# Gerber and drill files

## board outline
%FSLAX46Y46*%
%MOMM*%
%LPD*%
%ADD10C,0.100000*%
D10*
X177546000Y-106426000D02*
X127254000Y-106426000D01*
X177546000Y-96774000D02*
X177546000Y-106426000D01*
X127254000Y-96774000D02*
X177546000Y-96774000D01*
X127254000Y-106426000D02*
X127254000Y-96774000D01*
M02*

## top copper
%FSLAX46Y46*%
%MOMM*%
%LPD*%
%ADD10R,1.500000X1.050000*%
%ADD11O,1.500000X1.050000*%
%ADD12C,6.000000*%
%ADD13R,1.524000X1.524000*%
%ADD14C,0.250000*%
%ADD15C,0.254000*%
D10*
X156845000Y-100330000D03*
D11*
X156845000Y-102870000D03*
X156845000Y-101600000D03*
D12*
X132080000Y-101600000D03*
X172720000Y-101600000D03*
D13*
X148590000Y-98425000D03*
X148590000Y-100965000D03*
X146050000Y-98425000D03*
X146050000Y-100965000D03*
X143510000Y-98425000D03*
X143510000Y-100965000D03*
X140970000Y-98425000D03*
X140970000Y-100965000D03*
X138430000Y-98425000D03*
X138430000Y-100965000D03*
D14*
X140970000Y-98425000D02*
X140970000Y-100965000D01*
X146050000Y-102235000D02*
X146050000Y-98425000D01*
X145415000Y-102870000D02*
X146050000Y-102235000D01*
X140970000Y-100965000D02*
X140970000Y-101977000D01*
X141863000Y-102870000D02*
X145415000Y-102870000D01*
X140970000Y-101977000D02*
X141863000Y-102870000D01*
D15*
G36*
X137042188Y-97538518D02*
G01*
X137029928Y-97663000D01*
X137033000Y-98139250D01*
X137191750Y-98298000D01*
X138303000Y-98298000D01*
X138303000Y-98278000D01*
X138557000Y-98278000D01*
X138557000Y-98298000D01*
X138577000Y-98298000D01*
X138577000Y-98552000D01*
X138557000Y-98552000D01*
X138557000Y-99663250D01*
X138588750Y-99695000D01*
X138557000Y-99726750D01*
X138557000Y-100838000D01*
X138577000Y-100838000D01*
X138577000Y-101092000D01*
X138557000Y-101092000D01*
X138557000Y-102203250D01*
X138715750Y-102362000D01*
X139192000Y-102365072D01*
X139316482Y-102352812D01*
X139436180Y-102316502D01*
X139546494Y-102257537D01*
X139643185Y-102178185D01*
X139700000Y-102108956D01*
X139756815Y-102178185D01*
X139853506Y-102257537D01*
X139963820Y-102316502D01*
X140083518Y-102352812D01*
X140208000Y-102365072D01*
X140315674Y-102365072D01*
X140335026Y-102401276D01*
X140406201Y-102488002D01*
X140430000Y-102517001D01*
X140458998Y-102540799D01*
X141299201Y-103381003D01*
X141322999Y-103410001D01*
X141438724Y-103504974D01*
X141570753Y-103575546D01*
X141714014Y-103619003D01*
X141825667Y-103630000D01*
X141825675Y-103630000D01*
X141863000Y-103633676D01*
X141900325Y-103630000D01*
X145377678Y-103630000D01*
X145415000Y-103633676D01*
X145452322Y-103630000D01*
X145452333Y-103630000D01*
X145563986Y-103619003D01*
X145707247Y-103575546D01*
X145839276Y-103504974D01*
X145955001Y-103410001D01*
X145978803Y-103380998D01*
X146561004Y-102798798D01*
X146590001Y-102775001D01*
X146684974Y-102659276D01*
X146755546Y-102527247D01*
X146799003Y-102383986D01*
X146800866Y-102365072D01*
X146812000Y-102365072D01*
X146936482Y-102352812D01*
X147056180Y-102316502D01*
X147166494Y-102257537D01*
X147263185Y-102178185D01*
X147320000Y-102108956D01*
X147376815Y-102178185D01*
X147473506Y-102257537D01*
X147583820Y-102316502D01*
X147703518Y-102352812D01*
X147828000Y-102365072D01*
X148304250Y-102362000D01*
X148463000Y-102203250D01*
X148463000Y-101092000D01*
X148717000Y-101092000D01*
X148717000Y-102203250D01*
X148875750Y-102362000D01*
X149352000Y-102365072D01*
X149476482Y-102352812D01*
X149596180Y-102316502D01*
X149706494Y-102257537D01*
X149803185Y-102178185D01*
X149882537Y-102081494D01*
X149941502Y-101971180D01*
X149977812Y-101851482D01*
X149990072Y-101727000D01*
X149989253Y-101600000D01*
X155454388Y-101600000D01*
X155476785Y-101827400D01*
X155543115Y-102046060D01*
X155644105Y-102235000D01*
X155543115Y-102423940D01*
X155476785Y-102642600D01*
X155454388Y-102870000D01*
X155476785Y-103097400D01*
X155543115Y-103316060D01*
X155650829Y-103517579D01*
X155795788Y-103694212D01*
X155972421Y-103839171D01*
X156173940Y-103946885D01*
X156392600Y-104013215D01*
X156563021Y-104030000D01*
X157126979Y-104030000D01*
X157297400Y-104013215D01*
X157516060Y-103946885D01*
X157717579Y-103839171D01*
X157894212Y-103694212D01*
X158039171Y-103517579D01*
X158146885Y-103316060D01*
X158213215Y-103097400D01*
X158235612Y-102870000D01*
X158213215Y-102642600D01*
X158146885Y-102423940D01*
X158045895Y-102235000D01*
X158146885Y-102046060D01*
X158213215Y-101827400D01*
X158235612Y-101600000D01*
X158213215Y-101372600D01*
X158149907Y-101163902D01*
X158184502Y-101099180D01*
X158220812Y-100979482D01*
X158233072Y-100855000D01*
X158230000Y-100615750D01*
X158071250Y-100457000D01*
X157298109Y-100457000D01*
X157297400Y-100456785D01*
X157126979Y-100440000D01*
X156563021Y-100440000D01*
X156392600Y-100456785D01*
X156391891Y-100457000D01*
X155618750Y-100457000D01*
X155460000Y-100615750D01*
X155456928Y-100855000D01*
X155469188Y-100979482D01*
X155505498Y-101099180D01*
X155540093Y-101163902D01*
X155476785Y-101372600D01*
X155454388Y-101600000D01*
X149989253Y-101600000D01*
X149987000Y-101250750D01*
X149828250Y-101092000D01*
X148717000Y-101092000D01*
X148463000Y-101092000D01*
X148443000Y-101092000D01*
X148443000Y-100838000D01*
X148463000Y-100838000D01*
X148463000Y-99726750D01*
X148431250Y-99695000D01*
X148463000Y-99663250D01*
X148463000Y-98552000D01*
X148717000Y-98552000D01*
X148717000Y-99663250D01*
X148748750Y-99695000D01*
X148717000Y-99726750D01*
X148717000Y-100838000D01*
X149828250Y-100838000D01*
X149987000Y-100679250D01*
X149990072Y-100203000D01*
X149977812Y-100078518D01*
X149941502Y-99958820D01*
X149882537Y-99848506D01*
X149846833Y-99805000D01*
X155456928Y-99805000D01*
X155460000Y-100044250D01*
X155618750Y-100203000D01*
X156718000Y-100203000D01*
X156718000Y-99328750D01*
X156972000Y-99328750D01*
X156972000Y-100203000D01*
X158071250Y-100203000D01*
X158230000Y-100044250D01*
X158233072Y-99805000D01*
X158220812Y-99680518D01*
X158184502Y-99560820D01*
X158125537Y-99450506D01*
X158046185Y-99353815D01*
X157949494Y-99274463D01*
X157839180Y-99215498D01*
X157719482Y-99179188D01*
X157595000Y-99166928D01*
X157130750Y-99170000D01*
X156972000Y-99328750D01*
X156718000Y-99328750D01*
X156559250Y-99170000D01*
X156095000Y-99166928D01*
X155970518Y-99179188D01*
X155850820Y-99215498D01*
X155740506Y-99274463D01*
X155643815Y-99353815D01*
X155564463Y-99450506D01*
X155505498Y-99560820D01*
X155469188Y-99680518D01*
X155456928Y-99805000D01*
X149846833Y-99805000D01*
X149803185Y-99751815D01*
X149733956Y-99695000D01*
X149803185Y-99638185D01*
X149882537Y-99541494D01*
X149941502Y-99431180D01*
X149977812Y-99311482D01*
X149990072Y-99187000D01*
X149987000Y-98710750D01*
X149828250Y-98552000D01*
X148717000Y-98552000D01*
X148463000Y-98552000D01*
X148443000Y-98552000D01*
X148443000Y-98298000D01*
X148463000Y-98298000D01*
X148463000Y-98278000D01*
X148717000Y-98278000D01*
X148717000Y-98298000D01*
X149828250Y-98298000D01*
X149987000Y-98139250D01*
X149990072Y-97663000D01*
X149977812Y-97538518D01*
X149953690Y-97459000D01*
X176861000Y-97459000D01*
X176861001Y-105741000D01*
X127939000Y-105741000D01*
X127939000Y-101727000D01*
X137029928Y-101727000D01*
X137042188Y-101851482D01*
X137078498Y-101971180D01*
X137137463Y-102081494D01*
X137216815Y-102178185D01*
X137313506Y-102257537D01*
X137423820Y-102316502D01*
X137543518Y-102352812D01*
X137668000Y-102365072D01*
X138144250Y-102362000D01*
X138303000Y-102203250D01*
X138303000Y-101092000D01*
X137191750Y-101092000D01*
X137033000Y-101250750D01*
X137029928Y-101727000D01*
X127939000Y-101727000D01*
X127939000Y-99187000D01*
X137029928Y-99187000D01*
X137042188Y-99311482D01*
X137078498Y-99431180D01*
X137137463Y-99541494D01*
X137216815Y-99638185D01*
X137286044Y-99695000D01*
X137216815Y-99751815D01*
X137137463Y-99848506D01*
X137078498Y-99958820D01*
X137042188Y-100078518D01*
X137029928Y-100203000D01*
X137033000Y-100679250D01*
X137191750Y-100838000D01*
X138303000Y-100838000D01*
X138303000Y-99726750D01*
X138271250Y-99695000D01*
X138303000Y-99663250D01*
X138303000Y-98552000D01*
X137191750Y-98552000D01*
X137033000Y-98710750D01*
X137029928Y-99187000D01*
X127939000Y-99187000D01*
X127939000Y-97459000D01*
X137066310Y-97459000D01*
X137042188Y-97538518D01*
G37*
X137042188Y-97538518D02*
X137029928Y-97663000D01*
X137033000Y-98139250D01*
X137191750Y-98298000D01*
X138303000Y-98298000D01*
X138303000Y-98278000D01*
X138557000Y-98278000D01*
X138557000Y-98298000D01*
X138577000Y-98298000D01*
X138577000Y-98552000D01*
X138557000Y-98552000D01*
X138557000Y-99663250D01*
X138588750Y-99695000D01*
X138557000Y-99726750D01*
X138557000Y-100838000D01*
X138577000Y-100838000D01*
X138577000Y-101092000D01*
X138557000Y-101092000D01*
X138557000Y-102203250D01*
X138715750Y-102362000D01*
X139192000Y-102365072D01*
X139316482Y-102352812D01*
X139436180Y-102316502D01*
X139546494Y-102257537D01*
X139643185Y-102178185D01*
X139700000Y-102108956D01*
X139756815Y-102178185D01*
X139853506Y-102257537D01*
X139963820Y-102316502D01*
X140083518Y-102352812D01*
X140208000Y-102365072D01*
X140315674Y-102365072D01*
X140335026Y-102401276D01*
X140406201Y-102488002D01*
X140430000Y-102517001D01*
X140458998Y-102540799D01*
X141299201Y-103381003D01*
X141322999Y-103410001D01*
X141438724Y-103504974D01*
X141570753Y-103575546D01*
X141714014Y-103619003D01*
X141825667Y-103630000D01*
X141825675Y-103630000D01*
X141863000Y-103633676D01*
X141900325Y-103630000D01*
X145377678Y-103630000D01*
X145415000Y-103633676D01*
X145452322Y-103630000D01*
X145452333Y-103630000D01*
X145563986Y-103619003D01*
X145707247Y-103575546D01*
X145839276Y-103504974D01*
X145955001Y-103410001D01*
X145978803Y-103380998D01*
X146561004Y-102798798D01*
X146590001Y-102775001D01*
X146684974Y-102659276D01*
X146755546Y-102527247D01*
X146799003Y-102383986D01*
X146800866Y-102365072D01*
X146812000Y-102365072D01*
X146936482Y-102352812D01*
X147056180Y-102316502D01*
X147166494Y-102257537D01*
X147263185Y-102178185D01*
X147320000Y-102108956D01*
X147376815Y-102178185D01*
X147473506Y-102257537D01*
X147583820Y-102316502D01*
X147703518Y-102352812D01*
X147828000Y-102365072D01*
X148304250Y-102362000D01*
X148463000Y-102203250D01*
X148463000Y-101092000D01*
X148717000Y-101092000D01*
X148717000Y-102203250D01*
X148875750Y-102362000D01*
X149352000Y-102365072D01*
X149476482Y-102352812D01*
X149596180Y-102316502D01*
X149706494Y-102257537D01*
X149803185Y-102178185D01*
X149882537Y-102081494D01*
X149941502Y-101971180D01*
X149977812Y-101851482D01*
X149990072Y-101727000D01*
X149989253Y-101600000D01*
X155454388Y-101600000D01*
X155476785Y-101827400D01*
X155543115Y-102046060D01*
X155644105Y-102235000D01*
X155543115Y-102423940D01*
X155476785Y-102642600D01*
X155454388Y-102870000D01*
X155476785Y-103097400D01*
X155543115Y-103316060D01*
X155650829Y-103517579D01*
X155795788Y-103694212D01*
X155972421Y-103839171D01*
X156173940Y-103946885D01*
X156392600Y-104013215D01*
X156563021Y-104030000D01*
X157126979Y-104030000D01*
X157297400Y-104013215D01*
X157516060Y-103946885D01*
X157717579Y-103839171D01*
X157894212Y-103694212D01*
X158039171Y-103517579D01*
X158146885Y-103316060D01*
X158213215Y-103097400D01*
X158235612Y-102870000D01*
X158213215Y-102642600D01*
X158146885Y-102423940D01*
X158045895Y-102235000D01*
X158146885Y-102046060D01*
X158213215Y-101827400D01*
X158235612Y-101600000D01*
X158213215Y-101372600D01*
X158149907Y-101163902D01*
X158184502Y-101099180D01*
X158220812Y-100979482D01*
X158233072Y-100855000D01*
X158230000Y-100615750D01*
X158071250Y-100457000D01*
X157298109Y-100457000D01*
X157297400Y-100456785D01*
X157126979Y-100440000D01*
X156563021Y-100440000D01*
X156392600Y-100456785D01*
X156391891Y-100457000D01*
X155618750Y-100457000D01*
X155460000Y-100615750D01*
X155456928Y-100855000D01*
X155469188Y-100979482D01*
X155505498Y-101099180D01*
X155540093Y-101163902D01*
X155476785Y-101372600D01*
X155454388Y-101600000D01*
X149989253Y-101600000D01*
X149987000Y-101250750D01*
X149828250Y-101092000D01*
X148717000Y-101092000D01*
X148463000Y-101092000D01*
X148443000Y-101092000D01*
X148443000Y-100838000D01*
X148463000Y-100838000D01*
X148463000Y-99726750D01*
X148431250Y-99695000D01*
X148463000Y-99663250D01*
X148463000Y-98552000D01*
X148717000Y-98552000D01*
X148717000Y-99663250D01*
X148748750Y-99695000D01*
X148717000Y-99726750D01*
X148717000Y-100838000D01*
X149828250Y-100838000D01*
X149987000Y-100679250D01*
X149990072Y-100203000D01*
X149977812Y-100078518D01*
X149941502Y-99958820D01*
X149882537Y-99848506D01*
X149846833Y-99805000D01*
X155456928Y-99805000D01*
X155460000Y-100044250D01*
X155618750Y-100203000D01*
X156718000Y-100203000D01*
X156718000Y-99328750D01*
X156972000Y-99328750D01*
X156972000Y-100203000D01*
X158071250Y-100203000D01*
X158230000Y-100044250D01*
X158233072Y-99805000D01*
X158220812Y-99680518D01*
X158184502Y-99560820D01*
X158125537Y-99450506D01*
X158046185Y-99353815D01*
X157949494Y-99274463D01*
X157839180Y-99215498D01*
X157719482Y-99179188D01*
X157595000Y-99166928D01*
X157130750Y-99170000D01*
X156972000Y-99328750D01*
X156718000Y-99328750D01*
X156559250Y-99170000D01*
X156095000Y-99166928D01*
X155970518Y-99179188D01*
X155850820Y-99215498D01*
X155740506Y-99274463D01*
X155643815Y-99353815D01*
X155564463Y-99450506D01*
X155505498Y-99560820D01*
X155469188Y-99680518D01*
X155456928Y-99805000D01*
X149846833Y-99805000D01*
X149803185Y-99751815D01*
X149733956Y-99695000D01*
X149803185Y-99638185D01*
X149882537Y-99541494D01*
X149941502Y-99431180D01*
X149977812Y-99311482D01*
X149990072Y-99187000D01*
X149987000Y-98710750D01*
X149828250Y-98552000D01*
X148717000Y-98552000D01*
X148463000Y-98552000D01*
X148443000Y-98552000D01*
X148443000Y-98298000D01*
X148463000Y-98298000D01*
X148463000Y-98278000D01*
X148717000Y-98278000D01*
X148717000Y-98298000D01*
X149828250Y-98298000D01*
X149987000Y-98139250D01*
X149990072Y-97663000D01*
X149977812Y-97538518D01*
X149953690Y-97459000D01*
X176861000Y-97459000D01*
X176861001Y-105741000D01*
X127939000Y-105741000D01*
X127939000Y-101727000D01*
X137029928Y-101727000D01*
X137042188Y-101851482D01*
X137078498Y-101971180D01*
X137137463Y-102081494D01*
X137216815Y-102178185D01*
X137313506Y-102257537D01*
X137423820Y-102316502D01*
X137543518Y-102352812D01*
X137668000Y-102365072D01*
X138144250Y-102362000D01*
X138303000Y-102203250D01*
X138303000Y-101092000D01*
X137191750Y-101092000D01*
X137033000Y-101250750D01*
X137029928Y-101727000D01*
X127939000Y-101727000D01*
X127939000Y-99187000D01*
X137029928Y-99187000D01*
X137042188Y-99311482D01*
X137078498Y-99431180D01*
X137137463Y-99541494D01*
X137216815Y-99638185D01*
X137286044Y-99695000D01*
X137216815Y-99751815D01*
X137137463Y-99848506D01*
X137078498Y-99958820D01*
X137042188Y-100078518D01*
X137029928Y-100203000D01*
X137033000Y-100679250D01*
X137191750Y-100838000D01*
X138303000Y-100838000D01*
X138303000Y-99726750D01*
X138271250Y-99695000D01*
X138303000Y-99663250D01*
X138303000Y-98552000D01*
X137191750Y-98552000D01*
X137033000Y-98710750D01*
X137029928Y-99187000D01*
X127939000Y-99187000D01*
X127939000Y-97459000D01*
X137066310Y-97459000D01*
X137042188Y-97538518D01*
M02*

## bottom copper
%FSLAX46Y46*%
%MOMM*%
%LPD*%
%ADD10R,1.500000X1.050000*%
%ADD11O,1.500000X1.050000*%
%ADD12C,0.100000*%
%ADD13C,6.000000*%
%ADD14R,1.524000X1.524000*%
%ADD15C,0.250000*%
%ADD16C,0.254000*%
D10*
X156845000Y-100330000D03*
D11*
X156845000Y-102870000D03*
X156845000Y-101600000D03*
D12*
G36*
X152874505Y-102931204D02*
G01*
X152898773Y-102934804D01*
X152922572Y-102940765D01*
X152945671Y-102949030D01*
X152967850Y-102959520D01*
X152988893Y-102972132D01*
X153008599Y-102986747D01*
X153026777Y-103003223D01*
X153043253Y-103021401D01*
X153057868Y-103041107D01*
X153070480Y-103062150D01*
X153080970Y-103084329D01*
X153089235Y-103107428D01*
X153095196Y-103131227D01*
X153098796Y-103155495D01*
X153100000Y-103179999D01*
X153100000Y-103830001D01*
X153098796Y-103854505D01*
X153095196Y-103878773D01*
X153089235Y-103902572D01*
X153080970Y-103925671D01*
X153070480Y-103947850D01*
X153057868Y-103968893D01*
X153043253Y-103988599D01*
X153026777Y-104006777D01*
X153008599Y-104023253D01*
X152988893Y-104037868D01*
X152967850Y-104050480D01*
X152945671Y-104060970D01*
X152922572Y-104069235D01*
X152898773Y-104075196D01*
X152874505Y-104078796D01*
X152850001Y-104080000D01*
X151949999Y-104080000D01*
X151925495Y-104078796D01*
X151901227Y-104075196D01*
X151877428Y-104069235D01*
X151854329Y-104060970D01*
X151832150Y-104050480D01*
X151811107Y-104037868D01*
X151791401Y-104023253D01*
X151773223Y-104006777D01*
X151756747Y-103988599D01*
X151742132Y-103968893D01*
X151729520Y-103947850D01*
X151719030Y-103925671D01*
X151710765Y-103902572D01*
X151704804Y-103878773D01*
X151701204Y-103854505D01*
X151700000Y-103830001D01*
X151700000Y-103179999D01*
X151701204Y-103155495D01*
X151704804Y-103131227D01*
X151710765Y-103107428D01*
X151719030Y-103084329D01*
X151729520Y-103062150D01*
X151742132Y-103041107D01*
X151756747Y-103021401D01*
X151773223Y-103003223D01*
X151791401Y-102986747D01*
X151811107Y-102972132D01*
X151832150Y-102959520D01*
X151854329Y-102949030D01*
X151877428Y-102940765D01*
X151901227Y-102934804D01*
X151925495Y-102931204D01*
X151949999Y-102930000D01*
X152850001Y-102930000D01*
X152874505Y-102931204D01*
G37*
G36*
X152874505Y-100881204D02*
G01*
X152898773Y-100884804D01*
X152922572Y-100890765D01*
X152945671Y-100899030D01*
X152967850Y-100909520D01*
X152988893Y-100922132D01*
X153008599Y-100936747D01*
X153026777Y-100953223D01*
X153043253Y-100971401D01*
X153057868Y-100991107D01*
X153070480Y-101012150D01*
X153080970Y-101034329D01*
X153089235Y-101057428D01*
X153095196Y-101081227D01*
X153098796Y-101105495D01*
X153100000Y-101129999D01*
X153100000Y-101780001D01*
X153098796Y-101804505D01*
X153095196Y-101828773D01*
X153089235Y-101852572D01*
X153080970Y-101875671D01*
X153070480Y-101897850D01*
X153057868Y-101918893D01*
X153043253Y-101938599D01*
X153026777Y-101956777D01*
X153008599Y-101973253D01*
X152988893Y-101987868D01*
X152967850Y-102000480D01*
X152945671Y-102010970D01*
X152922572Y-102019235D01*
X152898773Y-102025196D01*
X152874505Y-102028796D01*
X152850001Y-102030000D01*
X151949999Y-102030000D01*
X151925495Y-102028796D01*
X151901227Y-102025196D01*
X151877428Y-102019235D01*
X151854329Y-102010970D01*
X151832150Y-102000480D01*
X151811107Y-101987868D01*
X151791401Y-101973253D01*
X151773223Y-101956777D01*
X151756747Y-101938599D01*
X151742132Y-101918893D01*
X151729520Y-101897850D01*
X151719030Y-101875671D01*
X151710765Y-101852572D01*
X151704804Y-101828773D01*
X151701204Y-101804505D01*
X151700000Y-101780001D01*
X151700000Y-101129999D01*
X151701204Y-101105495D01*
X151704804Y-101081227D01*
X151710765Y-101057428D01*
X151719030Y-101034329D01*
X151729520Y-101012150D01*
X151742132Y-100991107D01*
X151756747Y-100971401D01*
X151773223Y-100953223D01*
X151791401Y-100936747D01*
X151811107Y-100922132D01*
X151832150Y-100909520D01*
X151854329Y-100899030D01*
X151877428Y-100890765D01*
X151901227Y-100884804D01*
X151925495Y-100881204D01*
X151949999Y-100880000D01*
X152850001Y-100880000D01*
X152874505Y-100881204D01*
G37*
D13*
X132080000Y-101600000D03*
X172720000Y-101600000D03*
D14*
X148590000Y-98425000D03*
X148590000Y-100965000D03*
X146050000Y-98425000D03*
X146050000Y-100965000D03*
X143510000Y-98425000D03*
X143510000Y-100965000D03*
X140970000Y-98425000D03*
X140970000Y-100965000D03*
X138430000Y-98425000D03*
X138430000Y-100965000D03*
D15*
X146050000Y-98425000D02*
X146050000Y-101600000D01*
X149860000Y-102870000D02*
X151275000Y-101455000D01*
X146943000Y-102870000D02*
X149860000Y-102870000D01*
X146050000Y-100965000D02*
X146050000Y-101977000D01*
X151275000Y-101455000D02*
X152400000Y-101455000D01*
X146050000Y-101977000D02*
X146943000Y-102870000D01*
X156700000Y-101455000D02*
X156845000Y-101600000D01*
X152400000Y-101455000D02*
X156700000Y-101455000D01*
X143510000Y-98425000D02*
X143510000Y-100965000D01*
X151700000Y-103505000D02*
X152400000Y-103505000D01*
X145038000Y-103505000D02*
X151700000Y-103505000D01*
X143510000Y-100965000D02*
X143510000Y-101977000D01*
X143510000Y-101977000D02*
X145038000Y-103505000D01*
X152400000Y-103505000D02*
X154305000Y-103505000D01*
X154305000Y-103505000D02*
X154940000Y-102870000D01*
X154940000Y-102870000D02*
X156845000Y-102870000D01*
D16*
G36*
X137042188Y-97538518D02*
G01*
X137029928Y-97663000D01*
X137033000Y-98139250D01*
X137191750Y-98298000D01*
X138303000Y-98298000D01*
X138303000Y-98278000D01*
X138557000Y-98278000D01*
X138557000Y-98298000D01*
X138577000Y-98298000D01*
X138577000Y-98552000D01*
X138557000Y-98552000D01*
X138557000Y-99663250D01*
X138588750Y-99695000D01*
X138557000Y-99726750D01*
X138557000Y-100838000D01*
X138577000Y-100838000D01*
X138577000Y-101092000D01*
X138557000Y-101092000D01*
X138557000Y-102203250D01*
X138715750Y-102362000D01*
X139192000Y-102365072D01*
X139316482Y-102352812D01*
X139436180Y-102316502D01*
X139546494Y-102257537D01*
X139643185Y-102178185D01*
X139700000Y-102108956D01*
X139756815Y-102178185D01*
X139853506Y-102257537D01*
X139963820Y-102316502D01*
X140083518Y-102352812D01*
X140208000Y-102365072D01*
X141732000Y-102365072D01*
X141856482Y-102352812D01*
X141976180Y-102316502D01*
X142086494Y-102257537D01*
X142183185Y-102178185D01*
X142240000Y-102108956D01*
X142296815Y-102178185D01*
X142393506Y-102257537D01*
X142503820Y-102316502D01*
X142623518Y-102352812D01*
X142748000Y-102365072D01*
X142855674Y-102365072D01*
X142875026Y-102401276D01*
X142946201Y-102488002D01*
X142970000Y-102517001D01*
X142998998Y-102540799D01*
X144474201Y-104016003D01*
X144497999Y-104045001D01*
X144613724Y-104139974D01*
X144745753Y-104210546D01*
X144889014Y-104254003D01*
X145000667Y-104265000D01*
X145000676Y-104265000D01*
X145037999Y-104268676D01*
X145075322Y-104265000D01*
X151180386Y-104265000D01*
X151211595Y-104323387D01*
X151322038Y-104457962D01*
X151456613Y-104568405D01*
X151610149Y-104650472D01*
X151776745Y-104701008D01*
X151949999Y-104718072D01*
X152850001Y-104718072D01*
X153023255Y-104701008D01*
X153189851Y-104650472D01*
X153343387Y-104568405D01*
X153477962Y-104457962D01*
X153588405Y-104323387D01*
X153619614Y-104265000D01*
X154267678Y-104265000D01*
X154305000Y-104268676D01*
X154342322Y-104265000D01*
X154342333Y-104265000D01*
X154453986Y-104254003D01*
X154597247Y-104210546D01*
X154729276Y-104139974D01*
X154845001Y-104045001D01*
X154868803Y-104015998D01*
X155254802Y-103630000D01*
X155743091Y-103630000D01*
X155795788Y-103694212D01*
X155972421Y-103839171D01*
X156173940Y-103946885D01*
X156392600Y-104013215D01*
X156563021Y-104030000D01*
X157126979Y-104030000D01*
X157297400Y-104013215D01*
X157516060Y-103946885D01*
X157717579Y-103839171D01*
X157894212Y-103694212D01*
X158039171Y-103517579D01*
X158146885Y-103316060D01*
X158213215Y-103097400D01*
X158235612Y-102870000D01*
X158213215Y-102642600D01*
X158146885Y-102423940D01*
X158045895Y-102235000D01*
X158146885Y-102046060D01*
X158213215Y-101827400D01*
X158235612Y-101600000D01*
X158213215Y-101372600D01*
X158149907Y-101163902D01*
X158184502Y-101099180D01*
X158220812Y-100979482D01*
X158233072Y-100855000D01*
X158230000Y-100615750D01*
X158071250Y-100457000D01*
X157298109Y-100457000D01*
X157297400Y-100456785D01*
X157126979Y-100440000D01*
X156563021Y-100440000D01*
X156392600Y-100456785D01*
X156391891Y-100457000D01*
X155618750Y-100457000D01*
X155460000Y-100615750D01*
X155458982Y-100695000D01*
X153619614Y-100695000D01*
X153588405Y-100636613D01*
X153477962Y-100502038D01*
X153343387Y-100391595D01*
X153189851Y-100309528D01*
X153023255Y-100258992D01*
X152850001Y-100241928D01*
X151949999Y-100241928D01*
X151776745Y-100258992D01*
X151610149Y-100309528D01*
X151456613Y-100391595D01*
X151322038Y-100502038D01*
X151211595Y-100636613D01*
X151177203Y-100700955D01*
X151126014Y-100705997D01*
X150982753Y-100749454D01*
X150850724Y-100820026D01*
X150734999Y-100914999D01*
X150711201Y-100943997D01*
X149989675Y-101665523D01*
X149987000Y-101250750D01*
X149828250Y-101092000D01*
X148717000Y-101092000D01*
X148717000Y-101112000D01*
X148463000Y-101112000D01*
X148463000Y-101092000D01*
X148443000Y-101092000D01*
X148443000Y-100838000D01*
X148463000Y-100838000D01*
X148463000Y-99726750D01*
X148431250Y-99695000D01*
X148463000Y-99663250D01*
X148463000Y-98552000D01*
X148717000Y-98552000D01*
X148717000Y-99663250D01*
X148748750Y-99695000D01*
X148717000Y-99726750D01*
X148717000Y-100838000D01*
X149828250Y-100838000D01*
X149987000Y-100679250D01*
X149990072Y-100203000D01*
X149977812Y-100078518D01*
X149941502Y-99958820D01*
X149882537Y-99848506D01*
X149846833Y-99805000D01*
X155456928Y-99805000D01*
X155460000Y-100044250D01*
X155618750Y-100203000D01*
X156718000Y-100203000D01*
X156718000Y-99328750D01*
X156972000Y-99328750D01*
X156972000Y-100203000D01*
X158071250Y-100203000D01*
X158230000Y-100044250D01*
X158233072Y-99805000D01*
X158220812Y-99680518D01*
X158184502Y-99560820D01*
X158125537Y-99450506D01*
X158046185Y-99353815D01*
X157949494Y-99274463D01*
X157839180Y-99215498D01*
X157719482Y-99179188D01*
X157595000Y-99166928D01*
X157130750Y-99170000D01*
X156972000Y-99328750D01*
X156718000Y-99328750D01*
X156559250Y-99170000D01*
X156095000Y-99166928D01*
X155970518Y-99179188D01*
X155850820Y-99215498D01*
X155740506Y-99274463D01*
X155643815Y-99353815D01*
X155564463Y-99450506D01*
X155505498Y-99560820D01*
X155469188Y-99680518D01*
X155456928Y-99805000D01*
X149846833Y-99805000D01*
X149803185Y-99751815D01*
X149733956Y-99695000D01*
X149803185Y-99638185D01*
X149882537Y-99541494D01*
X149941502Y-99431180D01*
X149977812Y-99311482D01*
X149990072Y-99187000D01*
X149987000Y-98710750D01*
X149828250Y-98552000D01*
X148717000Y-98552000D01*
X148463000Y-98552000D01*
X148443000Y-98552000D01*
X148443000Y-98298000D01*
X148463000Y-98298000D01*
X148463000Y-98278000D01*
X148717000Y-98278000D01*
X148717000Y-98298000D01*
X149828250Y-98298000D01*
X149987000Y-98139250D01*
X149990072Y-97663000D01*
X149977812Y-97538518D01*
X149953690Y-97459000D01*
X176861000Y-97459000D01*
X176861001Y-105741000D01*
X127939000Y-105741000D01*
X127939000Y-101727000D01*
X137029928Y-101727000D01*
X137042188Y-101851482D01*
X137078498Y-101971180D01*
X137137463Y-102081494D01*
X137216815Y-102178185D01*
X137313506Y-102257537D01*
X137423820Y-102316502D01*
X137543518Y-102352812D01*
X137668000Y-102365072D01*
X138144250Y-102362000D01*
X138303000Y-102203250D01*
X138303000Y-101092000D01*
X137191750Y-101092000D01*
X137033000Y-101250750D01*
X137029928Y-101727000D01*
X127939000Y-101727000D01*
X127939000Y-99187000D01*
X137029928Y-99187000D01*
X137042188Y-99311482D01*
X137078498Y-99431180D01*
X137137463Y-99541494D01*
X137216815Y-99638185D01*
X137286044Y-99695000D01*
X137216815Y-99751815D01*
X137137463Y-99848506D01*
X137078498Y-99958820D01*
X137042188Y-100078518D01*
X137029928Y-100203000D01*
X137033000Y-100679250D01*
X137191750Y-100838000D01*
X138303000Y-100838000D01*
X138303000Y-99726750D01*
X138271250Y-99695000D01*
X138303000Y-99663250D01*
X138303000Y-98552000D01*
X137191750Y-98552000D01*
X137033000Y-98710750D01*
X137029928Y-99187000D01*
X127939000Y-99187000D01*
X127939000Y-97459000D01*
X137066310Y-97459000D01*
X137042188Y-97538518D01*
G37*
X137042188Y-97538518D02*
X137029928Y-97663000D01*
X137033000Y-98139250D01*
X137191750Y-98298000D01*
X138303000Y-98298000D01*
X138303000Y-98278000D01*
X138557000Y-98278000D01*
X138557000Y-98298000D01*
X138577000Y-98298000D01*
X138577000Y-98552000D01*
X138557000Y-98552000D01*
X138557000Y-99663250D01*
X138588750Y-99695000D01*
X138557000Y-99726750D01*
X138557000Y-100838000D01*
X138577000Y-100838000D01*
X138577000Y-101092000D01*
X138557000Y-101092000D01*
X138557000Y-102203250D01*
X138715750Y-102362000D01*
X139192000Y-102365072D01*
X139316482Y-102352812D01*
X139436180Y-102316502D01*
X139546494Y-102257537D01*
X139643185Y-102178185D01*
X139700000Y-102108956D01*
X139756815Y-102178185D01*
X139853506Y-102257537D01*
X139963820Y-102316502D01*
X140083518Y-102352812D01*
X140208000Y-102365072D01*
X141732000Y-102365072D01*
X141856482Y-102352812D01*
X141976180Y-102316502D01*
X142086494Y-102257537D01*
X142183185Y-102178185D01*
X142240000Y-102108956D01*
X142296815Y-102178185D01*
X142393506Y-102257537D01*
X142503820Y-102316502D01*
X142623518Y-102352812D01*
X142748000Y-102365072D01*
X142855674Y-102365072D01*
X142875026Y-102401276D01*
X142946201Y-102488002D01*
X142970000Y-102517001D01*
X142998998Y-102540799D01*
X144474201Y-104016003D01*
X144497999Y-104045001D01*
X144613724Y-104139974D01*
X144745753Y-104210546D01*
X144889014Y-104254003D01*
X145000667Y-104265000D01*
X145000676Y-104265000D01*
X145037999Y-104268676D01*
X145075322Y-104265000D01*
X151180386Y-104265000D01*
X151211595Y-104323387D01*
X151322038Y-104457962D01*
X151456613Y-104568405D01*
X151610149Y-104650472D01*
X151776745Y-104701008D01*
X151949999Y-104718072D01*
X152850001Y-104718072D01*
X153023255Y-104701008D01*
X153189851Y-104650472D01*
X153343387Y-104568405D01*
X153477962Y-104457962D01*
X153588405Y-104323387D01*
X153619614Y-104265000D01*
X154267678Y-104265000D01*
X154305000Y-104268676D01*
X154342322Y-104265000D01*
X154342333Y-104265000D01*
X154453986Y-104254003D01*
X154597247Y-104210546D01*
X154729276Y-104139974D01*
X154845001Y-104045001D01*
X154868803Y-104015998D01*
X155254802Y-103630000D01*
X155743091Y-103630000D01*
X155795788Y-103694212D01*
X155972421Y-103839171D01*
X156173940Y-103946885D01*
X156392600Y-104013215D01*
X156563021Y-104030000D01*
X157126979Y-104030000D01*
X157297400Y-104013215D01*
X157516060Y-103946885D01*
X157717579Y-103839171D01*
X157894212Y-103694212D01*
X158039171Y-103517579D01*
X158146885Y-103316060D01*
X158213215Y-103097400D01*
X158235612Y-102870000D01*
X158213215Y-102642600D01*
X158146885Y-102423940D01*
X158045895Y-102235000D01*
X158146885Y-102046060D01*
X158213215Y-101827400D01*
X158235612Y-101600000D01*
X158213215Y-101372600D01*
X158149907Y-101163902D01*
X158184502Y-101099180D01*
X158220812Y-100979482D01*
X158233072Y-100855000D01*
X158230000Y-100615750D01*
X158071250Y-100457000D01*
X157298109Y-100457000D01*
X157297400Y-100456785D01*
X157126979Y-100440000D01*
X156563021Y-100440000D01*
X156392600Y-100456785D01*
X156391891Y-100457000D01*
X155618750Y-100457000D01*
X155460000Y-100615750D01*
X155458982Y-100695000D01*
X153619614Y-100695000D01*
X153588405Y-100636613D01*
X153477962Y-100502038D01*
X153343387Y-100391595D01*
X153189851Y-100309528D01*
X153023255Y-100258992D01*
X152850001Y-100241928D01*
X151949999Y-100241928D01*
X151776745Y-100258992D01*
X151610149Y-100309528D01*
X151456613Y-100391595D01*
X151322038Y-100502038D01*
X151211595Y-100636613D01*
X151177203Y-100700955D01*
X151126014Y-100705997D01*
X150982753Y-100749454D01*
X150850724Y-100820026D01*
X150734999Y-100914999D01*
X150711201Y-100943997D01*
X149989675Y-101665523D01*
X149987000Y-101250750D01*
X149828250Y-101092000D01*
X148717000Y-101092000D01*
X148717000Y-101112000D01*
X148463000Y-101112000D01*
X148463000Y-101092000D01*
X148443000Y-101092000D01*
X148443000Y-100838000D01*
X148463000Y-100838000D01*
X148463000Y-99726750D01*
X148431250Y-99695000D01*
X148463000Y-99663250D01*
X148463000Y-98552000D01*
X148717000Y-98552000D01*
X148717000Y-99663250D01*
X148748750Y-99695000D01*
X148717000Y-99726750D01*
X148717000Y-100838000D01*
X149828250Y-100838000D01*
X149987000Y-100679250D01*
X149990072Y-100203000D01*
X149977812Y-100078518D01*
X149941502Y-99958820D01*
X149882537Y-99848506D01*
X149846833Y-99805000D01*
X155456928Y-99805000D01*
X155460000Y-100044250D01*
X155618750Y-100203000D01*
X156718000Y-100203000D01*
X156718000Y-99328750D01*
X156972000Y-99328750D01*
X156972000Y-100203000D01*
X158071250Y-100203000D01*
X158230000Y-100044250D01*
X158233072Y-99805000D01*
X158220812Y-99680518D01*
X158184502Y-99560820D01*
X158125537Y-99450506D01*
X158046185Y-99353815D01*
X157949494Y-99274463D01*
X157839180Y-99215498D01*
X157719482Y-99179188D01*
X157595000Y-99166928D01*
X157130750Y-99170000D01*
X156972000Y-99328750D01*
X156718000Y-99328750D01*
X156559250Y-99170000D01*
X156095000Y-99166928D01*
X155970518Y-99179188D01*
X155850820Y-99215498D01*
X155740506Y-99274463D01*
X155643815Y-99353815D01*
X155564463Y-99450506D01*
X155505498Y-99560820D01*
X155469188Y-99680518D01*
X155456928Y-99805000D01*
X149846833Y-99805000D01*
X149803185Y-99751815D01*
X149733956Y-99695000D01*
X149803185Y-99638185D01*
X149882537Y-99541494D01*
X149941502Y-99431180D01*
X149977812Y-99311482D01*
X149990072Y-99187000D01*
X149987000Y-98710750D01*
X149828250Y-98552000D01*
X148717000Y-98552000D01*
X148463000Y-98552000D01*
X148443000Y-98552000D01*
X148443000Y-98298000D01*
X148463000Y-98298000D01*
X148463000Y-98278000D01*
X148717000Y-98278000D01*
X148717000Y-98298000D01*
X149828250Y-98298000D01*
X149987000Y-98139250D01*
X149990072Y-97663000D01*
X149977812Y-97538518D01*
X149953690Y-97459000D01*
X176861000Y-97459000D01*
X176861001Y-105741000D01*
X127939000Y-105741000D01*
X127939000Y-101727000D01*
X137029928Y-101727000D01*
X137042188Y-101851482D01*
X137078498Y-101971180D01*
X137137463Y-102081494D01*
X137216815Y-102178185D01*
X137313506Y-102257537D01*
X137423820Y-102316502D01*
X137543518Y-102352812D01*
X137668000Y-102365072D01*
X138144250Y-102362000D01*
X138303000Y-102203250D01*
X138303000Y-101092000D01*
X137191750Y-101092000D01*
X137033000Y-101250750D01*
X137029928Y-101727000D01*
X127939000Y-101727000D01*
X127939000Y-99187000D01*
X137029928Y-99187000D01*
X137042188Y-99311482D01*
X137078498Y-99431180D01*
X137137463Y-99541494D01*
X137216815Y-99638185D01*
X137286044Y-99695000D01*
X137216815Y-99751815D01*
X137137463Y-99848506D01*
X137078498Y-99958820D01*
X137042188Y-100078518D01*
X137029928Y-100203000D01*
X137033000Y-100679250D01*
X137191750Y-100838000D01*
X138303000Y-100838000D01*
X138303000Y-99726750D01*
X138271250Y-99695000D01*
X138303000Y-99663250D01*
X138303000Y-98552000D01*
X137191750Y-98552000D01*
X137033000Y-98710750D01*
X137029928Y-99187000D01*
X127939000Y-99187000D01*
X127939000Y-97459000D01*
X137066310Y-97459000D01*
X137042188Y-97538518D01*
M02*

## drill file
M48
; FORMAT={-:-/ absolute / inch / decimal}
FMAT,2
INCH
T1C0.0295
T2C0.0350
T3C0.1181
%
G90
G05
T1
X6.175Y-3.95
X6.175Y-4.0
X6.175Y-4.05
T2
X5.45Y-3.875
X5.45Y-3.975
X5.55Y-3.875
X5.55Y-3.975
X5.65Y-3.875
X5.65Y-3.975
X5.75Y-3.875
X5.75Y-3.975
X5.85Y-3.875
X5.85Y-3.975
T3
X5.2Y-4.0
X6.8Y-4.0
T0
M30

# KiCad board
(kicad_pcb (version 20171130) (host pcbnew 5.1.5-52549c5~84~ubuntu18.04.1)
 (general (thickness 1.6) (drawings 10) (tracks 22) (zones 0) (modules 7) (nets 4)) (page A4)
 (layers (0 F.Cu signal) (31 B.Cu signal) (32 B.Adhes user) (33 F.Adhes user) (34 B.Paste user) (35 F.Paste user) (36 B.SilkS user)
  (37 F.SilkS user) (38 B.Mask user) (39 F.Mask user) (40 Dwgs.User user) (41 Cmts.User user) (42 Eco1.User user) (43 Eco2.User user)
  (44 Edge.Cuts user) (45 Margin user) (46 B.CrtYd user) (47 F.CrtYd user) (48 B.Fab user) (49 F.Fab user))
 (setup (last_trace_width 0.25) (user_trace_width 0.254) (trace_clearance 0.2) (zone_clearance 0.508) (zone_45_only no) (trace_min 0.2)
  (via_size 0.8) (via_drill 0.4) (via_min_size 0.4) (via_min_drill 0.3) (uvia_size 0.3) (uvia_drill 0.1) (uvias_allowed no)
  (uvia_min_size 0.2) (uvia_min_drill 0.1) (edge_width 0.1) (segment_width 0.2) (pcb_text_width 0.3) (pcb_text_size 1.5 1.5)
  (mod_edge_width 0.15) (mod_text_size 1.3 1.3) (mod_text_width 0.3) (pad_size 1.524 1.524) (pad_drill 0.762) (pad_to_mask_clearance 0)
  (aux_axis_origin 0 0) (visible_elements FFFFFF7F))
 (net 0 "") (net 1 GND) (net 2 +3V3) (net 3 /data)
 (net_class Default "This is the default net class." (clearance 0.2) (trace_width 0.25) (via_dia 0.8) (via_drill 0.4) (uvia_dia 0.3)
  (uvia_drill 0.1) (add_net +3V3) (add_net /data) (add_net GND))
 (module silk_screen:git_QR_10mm (layer B.Cu) (at 163.576 101.6)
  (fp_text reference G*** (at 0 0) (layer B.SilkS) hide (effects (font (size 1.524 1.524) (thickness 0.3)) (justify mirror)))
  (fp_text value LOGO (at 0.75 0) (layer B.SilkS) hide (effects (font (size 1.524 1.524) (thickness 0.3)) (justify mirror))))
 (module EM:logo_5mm (layer F.Cu) (at 164.465 101.6 90)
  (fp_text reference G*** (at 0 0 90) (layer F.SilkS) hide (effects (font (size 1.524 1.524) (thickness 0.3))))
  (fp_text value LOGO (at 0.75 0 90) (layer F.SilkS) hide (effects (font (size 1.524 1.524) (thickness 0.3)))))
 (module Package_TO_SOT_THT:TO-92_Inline (layer F.Cu) (at 156.845 100.33 270)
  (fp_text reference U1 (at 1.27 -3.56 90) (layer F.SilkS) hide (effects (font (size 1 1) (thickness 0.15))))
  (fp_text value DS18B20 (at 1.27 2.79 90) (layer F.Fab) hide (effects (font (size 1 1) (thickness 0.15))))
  (pad 1 thru_hole rect (at 0 0 270) (size 1.05 1.5) (drill 0.75) (layers *.Cu *.Mask) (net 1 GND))
  (pad 3 thru_hole oval (at 2.54 0 270) (size 1.05 1.5) (drill 0.75) (layers *.Cu *.Mask) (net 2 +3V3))
  (pad 2 thru_hole oval (at 1.27 0 270) (size 1.05 1.5) (drill 0.75) (layers *.Cu *.Mask) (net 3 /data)))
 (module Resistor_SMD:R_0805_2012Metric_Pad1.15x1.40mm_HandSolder (layer B.Cu) (at 152.4 102.48 270)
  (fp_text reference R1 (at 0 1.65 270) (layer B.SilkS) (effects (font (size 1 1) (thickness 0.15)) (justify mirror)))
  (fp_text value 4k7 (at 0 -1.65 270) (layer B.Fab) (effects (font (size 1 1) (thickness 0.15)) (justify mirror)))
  (pad 2 smd roundrect (at 1.025 0 270) (size 1.15 1.4) (layers B.Cu B.Paste B.Mask) (roundrect_rratio 0.217391) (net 2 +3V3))
  (pad 1 smd roundrect (at -1.025 0 270) (size 1.15 1.4) (layers B.Cu B.Paste B.Mask) (roundrect_rratio 0.217391) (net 3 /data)))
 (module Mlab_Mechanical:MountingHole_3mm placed (layer F.Cu) (at 132.08 101.6)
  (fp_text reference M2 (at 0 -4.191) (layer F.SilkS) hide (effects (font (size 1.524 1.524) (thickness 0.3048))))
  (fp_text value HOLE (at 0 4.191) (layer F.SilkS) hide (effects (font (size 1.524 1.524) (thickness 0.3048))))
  (pad 1 thru_hole circle (at 0 0) (size 6 6) (drill 3) (layers *.Cu *.Adhes *.Mask) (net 1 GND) (clearance 1) (zone_connect 2)))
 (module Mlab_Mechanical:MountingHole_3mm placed (layer F.Cu) (at 172.72 101.6)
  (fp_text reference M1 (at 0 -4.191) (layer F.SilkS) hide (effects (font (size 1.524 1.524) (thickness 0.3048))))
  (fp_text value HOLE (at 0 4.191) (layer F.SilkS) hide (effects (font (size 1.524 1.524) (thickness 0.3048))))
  (pad 1 thru_hole circle (at 0 0) (size 6 6) (drill 3) (layers *.Cu *.Adhes *.Mask) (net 1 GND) (clearance 1) (zone_connect 2)))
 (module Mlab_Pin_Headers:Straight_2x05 (layer F.Cu) (at 143.51 99.695 90)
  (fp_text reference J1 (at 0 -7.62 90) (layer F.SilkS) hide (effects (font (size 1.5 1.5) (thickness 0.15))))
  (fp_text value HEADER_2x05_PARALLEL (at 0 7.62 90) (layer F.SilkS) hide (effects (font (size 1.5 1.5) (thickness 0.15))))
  (pad 10 thru_hole rect (at 1.27 5.08 90) (size 1.524 1.524) (drill 0.889) (layers *.Cu *.Mask F.SilkS) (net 1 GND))
  (pad 9 thru_hole rect (at -1.27 5.08 90) (size 1.524 1.524) (drill 0.889) (layers *.Cu *.Mask F.SilkS) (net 1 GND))
  (pad 8 thru_hole rect (at 1.27 2.54 90) (size 1.524 1.524) (drill 0.889) (layers *.Cu *.Mask F.SilkS) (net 3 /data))
  (pad 7 thru_hole rect (at -1.27 2.54 90) (size 1.524 1.524) (drill 0.889) (layers *.Cu *.Mask F.SilkS) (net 3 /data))
  (pad 6 thru_hole rect (at 1.27 0 90) (size 1.524 1.524) (drill 0.889) (layers *.Cu *.Mask F.SilkS) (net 2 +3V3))
  (pad 5 thru_hole rect (at -1.27 0 90) (size 1.524 1.524) (drill 0.889) (layers *.Cu *.Mask F.SilkS) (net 2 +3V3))
  (pad 4 thru_hole rect (at 1.27 -2.54 90) (size 1.524 1.524) (drill 0.889) (layers *.Cu *.Mask F.SilkS) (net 3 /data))
  (pad 3 thru_hole rect (at -1.27 -2.54 90) (size 1.524 1.524) (drill 0.889) (layers *.Cu *.Mask F.SilkS) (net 3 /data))
  (pad 2 thru_hole rect (at 1.27 -5.08 90) (size 1.524 1.524) (drill 0.889) (layers *.Cu *.Mask F.SilkS) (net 1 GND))
  (pad 1 thru_hole rect (at -1.27 -5.08 90) (size 1.524 1.524) (drill 0.889) (layers *.Cu *.Mask F.SilkS) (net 1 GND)))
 (gr_line (start 177.546 106.426) (end 127.254 106.426) (layer Edge.Cuts) (width 0.1))
 (gr_line (start 177.546 96.774) (end 177.546 106.426) (layer Edge.Cuts) (width 0.1))
 (gr_line (start 127.254 96.774) (end 177.546 96.774) (layer Edge.Cuts) (width 0.1))
 (gr_line (start 127.254 106.426) (end 127.254 96.774) (layer Edge.Cuts) (width 0.1))
 (segment (start 140.97 98.425) (end 140.97 100.965) (width 0.25) (layer F.Cu) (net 3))
 (segment (start 146.05 102.235) (end 146.05 98.425) (width 0.25) (layer F.Cu) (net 3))
 (segment (start 145.415 102.87) (end 146.05 102.235) (width 0.25) (layer F.Cu) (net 3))
 (segment (start 140.97 100.965) (end 140.97 101.977) (width 0.25) (layer F.Cu) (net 3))
 (segment (start 141.863 102.87) (end 145.415 102.87) (width 0.25) (layer F.Cu) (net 3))
 (segment (start 140.97 101.977) (end 141.863 102.87) (width 0.25) (layer F.Cu) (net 3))
 (segment (start 146.05 98.425) (end 146.05 101.6) (width 0.25) (layer B.Cu) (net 3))
 (segment (start 149.86 102.87) (end 151.275 101.455) (width 0.25) (layer B.Cu) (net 3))
 (segment (start 146.943 102.87) (end 149.86 102.87) (width 0.25) (layer B.Cu) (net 3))
 (segment (start 146.05 100.965) (end 146.05 101.977) (width 0.25) (layer B.Cu) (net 3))
 (segment (start 151.275 101.455) (end 152.4 101.455) (width 0.25) (layer B.Cu) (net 3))
 (segment (start 146.05 101.977) (end 146.943 102.87) (width 0.25) (layer B.Cu) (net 3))
 (segment (start 156.7 101.455) (end 156.845 101.6) (width 0.25) (layer B.Cu) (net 3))
 (segment (start 152.4 101.455) (end 156.7 101.455) (width 0.25) (layer B.Cu) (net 3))
 (segment (start 143.51 98.425) (end 143.51 100.965) (width 0.25) (layer B.Cu) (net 2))
 (segment (start 151.7 103.505) (end 152.4 103.505) (width 0.25) (layer B.Cu) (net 2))
 (segment (start 145.038 103.505) (end 151.7 103.505) (width 0.25) (layer B.Cu) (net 2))
 (segment (start 143.51 100.965) (end 143.51 101.977) (width 0.25) (layer B.Cu) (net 2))
 (segment (start 143.51 101.977) (end 145.038 103.505) (width 0.25) (layer B.Cu) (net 2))
 (segment (start 152.4 103.505) (end 154.305 103.505) (width 0.25) (layer B.Cu) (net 2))
 (segment (start 154.305 103.505) (end 154.94 102.87) (width 0.25) (layer B.Cu) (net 2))
 (segment (start 154.94 102.87) (end 156.845 102.87) (width 0.25) (layer B.Cu) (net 2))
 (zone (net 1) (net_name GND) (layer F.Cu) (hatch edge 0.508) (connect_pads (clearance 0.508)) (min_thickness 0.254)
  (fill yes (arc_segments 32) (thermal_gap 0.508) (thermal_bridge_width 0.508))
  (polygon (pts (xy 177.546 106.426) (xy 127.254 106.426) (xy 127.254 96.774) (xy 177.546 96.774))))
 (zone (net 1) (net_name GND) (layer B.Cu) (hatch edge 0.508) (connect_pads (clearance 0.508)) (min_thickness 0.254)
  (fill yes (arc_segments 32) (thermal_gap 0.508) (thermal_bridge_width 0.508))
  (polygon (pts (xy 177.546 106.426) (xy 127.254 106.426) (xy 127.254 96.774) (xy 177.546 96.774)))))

